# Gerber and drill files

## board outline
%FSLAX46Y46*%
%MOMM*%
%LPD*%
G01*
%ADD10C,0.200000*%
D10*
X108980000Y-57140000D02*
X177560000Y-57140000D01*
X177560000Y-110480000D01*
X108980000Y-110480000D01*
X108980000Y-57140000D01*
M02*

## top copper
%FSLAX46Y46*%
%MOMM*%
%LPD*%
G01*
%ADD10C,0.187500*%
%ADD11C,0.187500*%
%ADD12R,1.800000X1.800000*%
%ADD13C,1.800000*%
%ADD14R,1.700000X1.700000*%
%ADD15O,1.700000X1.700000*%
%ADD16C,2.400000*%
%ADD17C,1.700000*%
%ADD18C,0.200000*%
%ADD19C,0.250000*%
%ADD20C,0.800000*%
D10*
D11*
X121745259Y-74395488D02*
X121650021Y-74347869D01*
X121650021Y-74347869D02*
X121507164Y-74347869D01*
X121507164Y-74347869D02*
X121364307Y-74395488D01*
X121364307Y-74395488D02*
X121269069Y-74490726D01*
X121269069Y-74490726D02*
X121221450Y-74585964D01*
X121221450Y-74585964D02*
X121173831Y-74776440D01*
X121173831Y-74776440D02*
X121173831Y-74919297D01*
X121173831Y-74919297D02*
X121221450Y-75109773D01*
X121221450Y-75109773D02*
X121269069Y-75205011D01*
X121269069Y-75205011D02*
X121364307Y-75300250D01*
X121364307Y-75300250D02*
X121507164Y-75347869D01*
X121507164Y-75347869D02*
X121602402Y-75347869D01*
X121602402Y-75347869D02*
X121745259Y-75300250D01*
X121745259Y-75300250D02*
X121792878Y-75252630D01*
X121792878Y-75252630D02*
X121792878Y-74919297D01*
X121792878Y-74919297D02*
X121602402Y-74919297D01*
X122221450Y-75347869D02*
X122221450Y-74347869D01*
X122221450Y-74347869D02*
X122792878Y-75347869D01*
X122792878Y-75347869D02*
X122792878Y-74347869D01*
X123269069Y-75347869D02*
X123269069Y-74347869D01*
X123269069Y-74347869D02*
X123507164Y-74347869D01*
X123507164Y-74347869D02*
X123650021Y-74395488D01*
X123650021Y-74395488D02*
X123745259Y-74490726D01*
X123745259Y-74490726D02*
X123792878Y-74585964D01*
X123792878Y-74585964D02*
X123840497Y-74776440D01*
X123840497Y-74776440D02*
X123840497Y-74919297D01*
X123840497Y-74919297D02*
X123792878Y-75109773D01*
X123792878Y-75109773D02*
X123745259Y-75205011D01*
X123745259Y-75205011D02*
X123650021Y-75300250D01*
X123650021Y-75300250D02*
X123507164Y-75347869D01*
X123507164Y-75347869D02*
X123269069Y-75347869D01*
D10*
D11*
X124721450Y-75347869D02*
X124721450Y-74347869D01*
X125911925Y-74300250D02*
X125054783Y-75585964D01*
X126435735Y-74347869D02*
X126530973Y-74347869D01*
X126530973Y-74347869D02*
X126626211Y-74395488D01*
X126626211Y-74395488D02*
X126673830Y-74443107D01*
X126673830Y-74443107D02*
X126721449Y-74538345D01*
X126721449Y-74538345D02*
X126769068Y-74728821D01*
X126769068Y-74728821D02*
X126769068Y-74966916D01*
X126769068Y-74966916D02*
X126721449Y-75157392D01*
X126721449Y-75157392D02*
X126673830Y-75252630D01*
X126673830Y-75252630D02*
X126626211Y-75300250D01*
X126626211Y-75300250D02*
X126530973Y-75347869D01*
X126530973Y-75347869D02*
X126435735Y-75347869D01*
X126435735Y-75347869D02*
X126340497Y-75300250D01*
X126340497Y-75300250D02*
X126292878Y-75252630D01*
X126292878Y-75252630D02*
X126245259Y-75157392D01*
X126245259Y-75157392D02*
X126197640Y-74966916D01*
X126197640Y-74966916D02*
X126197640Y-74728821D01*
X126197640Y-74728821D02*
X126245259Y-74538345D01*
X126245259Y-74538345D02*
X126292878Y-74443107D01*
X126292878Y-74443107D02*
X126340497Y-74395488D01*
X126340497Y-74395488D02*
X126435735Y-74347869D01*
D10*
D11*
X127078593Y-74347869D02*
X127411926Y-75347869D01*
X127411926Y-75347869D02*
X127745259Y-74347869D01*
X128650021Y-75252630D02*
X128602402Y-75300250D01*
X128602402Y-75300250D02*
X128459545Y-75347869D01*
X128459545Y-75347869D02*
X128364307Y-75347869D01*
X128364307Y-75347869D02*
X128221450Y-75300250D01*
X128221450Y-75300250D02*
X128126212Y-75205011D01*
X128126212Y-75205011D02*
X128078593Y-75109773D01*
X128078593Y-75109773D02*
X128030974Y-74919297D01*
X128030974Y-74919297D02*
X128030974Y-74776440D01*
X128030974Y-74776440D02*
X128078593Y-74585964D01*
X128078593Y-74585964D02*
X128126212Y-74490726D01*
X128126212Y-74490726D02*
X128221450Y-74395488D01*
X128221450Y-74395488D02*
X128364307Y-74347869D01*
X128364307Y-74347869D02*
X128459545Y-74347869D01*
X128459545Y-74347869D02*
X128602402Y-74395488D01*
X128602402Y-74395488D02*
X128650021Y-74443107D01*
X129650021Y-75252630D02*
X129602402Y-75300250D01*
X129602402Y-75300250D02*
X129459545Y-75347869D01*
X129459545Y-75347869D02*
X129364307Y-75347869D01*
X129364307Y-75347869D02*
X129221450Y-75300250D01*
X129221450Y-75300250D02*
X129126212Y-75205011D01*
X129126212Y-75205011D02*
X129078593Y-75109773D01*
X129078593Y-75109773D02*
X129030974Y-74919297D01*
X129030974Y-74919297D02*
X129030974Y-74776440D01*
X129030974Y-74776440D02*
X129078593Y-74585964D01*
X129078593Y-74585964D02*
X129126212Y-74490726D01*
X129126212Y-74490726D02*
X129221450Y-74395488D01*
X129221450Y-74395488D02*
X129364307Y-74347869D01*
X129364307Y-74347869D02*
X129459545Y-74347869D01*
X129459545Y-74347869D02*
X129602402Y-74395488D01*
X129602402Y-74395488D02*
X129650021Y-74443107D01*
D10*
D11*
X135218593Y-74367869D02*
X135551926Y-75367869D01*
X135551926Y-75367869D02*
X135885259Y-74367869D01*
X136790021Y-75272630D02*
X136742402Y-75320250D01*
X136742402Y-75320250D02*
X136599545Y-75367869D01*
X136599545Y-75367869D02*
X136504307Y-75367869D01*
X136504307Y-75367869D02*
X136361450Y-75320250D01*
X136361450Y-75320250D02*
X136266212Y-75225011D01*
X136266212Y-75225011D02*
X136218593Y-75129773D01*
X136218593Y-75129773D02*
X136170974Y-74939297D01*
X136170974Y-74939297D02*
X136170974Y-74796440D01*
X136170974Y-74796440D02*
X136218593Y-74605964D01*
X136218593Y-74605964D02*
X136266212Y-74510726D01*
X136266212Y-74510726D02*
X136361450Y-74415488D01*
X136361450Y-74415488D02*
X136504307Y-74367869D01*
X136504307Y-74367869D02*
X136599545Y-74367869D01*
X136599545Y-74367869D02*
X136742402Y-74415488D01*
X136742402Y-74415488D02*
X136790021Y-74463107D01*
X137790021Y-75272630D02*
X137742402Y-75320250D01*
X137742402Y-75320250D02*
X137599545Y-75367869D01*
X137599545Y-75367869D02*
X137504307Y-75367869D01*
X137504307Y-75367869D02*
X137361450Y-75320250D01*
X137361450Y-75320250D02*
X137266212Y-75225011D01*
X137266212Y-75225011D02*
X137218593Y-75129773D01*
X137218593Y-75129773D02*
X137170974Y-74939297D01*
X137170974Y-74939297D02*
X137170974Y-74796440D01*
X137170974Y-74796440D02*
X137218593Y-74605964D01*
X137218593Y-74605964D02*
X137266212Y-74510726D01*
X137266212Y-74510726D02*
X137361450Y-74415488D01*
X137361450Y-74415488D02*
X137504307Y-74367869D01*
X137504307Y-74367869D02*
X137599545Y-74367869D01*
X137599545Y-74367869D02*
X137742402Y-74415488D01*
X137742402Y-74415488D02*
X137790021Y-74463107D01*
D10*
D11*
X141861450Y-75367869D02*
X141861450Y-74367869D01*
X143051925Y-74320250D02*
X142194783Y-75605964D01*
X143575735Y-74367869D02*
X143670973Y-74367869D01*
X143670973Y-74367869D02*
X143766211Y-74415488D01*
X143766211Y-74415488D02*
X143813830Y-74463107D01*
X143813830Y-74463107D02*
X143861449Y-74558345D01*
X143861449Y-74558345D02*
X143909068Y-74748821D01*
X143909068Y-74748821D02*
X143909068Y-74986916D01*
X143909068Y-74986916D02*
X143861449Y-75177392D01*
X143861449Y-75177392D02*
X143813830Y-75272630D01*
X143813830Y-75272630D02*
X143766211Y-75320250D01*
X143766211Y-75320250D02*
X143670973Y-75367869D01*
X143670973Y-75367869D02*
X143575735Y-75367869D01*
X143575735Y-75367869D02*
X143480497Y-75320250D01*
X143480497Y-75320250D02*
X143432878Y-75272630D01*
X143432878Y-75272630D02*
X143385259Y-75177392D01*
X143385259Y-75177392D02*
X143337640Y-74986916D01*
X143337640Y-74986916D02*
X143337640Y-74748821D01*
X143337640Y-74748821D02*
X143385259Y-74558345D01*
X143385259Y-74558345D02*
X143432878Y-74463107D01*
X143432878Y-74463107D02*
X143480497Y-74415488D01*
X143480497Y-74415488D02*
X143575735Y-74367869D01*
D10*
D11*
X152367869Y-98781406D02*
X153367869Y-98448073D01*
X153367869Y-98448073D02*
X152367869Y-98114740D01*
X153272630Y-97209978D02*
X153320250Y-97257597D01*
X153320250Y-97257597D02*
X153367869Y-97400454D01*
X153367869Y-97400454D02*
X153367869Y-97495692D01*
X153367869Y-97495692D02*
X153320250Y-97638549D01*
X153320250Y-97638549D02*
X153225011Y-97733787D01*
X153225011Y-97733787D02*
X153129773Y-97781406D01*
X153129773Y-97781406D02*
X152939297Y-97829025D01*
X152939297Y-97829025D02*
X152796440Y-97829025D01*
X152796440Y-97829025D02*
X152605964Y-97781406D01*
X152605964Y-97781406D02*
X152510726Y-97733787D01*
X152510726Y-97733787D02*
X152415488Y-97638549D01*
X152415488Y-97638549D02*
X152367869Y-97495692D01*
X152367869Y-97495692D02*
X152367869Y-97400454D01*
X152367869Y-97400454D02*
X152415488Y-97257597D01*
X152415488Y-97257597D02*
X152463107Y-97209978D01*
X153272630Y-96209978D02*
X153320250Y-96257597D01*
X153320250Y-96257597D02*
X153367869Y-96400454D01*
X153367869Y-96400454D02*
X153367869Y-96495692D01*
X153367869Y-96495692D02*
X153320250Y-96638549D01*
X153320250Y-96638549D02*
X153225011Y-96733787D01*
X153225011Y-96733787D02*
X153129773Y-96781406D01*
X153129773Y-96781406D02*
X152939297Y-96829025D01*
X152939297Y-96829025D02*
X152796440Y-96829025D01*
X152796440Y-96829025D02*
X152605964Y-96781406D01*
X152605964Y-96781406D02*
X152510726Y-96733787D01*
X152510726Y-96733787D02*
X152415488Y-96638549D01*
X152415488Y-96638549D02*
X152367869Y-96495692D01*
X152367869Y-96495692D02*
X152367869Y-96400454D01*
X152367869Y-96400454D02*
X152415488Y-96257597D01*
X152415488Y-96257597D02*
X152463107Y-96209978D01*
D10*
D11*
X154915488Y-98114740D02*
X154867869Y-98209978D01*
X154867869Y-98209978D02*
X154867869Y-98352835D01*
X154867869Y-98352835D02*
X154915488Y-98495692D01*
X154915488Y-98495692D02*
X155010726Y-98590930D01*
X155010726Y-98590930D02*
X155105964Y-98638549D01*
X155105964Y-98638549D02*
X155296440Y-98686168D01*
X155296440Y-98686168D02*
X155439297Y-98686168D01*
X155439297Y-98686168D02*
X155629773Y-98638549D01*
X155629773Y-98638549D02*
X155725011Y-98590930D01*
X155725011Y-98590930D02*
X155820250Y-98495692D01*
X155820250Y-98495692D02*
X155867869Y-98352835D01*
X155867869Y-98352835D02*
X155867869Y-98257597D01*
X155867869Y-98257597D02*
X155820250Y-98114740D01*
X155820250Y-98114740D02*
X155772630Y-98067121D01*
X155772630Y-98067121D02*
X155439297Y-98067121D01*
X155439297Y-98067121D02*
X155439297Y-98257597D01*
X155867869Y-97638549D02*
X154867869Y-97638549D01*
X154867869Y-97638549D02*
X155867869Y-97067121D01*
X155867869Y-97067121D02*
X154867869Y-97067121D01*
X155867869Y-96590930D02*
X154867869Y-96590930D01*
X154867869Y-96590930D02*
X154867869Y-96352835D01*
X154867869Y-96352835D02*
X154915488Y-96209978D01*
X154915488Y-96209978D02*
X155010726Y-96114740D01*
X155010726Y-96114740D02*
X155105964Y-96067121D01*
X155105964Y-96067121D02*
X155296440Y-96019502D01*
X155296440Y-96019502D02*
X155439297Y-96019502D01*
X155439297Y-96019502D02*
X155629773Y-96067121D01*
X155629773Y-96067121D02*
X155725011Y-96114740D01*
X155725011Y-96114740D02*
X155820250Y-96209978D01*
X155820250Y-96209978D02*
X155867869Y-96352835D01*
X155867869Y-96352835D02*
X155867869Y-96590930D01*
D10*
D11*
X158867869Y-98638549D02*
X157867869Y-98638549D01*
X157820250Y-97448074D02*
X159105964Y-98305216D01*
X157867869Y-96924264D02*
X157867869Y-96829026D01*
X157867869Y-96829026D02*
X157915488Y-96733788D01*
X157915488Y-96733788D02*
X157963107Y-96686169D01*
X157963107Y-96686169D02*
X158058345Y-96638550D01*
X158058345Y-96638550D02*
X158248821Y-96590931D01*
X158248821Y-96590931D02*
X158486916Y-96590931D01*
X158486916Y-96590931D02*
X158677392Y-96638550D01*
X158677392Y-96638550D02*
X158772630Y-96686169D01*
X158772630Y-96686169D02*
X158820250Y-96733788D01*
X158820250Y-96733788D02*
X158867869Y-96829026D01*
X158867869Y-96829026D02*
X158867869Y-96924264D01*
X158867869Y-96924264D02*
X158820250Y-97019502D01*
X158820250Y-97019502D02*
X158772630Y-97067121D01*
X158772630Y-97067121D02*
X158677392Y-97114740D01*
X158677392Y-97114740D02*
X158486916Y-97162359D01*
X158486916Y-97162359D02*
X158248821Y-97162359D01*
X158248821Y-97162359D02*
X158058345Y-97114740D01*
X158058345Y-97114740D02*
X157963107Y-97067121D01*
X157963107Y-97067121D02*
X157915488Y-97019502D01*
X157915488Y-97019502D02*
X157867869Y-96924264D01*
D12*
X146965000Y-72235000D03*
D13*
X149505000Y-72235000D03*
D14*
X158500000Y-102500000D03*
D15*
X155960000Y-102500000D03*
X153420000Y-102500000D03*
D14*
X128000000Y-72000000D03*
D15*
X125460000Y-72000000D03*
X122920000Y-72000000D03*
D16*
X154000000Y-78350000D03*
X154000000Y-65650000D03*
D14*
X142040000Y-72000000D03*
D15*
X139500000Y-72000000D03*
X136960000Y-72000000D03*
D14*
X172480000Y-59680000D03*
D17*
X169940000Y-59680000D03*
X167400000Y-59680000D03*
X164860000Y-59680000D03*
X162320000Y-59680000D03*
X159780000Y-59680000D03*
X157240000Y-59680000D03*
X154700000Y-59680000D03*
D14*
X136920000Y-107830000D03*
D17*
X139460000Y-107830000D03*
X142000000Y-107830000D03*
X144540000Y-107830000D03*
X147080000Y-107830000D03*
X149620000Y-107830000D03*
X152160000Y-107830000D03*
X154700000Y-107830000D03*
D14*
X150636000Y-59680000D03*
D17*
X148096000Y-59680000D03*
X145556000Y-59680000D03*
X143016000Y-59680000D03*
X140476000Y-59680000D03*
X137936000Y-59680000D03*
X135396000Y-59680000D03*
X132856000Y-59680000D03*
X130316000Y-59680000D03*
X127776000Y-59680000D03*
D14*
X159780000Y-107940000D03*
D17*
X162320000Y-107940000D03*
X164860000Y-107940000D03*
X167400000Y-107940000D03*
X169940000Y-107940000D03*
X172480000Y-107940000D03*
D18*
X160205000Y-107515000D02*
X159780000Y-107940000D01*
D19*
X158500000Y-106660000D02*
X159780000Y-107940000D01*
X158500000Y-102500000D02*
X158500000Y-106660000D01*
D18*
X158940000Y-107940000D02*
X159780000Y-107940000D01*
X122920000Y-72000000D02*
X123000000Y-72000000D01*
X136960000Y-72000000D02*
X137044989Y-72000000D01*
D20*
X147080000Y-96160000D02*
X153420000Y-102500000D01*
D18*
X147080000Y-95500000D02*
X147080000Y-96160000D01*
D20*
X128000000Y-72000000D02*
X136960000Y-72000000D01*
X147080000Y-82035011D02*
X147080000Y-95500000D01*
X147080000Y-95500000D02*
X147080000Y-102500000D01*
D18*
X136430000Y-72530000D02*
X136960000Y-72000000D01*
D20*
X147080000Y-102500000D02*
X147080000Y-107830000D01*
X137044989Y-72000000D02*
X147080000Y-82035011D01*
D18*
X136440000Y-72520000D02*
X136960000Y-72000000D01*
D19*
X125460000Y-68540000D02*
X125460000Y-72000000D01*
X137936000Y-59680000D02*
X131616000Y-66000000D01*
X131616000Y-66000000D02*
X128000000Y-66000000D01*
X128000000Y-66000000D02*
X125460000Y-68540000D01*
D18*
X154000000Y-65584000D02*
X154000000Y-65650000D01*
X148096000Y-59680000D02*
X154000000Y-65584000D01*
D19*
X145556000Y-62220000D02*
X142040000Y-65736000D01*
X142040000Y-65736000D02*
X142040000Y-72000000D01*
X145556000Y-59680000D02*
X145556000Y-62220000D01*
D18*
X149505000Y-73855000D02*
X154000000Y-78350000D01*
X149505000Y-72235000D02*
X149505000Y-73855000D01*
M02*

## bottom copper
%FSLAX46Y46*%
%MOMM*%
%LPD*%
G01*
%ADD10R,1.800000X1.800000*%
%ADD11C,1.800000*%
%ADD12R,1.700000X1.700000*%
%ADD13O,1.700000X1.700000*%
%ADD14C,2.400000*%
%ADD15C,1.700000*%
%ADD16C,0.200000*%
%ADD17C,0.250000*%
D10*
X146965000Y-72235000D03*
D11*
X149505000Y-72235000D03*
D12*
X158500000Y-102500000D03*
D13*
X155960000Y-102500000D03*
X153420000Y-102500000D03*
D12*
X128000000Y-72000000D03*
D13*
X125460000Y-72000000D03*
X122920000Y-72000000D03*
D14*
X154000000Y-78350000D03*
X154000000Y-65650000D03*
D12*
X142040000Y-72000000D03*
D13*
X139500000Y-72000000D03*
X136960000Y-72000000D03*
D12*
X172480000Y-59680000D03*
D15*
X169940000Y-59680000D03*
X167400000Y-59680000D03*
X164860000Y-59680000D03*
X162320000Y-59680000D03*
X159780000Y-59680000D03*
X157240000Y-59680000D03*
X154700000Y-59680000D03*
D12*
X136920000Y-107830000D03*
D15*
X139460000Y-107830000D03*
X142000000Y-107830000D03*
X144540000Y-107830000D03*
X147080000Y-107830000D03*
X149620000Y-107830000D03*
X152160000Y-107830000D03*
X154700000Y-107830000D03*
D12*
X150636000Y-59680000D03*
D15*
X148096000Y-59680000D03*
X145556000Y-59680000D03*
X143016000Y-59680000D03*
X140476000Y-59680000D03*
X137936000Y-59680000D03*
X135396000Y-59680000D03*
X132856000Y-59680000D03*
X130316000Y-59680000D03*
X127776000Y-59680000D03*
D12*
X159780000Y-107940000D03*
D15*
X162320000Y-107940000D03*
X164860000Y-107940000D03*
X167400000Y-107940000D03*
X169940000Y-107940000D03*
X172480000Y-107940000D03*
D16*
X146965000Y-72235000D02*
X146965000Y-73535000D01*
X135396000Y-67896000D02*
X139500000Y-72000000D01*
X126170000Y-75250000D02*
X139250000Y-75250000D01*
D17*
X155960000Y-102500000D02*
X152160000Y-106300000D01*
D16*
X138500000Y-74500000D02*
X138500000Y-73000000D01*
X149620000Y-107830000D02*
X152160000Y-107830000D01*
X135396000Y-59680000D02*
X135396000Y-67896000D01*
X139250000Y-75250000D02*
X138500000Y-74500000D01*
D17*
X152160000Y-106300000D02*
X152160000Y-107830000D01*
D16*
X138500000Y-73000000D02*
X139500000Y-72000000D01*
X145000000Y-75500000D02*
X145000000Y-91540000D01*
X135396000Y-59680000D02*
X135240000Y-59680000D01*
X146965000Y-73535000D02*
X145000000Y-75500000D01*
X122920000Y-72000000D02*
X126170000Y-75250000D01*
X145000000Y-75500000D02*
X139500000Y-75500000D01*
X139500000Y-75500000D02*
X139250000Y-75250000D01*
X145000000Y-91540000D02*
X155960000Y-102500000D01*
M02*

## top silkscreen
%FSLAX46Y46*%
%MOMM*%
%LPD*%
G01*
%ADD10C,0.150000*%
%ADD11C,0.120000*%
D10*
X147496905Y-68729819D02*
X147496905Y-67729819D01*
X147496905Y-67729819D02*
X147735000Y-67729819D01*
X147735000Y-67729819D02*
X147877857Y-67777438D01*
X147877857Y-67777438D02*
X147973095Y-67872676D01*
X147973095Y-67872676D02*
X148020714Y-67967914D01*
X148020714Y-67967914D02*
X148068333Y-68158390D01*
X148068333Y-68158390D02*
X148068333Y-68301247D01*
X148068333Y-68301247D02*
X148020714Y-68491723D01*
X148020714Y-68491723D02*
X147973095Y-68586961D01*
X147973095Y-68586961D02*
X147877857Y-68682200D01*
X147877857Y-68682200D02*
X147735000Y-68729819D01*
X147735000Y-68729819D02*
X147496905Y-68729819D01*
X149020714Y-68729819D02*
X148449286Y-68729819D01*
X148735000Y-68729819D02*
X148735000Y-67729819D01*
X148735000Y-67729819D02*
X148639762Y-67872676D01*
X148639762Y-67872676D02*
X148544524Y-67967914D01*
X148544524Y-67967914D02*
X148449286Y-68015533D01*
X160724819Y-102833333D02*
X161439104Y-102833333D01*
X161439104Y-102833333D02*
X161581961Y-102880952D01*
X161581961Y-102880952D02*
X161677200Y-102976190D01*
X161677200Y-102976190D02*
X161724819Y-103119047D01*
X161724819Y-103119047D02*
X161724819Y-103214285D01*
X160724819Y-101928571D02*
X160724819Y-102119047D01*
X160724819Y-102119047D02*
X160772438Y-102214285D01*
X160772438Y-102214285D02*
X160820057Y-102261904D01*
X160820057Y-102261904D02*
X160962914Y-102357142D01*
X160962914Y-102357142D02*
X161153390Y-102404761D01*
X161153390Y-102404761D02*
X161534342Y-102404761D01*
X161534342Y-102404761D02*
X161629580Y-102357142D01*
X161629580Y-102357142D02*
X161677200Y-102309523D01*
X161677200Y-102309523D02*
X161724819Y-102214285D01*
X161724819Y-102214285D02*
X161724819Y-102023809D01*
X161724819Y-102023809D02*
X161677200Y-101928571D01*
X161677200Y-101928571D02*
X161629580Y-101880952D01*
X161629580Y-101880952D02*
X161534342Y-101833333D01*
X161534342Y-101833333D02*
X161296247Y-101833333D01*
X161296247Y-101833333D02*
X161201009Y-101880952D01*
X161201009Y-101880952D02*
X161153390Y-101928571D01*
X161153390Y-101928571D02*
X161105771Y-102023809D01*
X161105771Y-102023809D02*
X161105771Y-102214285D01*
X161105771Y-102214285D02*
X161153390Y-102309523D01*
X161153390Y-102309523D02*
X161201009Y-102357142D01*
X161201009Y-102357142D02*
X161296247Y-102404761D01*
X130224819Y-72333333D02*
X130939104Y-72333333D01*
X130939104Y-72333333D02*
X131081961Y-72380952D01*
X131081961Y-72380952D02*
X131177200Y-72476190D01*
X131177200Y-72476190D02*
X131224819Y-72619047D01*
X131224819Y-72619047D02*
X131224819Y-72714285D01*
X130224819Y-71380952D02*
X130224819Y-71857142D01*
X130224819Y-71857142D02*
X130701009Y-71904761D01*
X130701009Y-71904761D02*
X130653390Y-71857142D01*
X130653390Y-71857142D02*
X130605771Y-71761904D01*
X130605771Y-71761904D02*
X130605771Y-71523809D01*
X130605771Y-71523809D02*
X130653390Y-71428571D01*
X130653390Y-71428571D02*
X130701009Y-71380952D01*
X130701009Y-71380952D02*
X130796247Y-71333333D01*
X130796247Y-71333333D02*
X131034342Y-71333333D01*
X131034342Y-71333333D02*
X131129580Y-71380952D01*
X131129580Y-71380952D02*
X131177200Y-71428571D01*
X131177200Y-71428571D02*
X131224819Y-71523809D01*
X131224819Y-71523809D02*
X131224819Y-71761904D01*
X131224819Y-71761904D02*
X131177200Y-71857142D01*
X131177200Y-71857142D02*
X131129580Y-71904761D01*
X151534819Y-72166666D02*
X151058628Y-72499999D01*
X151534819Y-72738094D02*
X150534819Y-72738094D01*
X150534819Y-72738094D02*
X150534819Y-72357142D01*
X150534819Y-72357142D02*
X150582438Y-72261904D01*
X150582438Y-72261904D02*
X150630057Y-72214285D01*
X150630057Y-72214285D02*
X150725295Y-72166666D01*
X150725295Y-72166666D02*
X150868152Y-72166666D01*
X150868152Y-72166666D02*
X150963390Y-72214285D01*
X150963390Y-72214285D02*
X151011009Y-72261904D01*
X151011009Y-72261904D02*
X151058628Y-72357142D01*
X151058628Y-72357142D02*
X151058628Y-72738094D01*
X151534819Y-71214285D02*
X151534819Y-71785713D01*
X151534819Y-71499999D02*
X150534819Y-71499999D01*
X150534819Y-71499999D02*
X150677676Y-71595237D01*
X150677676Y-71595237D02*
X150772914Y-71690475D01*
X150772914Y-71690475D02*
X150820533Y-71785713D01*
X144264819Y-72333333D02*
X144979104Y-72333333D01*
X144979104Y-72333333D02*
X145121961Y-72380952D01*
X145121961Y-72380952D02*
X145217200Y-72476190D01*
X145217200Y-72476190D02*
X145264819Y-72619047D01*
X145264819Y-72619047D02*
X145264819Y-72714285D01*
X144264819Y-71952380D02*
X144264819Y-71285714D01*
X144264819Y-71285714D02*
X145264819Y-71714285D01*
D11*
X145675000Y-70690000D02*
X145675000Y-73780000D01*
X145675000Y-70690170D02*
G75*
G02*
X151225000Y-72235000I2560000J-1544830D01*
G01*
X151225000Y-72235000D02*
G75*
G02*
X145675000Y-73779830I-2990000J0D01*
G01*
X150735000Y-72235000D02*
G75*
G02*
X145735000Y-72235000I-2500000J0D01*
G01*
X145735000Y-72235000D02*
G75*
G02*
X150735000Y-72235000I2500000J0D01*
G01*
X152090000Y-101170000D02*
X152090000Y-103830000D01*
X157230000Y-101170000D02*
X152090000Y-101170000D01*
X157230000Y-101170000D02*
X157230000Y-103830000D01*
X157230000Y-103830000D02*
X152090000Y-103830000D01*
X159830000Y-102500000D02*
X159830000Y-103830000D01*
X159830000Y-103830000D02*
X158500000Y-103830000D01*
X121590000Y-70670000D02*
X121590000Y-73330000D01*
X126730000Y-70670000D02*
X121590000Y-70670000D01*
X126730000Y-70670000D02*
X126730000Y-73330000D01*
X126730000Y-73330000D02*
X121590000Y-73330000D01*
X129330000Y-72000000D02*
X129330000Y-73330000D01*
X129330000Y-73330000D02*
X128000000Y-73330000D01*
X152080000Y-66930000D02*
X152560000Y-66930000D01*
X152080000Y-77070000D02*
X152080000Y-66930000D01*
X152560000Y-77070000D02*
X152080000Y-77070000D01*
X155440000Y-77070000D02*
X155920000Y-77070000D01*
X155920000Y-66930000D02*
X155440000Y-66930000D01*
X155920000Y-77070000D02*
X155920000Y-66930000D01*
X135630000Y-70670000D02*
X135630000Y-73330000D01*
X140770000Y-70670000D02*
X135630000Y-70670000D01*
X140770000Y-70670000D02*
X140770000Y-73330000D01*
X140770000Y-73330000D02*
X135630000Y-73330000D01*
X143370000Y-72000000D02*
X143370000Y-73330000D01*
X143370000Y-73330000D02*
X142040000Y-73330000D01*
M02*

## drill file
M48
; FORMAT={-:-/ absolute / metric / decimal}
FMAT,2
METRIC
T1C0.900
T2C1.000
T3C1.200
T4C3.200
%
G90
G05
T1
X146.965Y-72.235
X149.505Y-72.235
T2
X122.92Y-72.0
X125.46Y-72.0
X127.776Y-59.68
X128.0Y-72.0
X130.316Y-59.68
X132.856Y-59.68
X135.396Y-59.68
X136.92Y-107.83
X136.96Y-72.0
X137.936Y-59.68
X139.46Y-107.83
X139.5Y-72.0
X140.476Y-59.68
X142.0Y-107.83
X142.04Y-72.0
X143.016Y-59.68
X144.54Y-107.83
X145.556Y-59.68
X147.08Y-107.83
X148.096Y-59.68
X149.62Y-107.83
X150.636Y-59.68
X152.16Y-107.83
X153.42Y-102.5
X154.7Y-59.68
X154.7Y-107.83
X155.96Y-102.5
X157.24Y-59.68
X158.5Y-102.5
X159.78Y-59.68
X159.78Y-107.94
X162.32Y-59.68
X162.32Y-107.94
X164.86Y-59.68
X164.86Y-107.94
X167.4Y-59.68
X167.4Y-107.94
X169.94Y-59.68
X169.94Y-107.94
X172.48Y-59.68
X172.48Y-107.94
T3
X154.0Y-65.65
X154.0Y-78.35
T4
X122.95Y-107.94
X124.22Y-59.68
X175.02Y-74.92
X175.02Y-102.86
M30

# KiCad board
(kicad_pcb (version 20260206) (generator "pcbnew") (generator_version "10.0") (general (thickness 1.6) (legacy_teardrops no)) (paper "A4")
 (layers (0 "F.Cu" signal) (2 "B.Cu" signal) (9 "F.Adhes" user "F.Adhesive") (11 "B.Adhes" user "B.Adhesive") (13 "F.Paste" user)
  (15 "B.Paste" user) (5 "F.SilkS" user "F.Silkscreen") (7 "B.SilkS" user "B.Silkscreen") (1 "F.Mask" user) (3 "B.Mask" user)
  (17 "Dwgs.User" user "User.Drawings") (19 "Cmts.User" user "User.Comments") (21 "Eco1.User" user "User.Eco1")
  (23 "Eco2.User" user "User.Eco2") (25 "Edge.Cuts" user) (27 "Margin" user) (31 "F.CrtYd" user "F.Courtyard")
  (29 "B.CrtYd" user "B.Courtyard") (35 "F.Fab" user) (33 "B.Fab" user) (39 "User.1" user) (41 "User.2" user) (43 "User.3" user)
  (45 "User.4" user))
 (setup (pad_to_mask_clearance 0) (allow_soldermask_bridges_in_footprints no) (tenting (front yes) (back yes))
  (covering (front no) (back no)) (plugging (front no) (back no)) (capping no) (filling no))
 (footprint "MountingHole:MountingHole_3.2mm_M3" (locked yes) (layer "F.Cu") (at 175.01997 102.860094)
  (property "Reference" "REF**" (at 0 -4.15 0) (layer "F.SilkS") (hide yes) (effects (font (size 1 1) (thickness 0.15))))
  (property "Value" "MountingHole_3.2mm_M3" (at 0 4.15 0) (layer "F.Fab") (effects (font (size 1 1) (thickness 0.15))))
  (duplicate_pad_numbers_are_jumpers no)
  (pad "" np_thru_hole circle (at 0 0) (size 3.2 3.2) (drill 3.2) (layers "*.Cu" "*.Mask")))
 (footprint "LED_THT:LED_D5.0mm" (layer "F.Cu") (at 146.965 72.235)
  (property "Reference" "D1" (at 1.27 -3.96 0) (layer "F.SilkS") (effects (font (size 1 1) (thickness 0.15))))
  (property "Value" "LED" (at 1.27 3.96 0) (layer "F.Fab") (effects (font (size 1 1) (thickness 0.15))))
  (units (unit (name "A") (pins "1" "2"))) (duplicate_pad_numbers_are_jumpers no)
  (fp_line (start -1.29 -1.545) (end -1.29 1.545) (stroke (width 0.12) (type solid)) (layer "F.SilkS"))
  (fp_arc (start -1.29 -1.54483) (mid 2.071779 -2.880495) (end 4.26 0) (stroke (width 0.12) (type solid)) (layer "F.SilkS"))
  (fp_arc (start 4.26 0) (mid 2.071779 2.880495) (end -1.29 1.54483) (stroke (width 0.12) (type solid)) (layer "F.SilkS"))
  (fp_circle (center 1.27 0) (end 3.77 0) (stroke (width 0.12) (type solid)) (fill no) (layer "F.SilkS"))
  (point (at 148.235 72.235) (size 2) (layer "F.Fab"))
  (pad "1" thru_hole rect (at 0 0) (size 1.8 1.8) (drill 0.9) (layers "*.Cu" "*.Mask") (remove_unused_layers no) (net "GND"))
  (pad "2" thru_hole circle (at 2.54 0) (size 1.8 1.8) (drill 0.9) (layers "*.Cu" "*.Mask") (remove_unused_layers no) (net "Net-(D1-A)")))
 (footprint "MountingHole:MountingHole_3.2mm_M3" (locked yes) (layer "F.Cu") (at 122.94997 107.940094)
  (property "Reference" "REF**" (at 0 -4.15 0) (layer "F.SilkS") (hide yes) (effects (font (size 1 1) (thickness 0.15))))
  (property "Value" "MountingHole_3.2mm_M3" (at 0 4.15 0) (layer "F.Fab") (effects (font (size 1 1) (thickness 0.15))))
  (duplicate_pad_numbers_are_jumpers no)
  (pad "" np_thru_hole circle (at 0 0) (size 3.2 3.2) (drill 3.2) (layers "*.Cu" "*.Mask")))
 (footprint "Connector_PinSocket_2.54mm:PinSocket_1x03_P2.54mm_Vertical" (layer "F.Cu") (at 158.5 102.5 -90)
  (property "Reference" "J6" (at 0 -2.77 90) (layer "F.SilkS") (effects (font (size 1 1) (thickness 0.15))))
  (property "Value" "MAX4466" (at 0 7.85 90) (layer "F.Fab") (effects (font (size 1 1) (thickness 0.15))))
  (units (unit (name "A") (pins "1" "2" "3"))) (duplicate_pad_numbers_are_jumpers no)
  (fp_line (start -1.33 6.41) (end 1.33 6.41) (stroke (width 0.12) (type solid)) (layer "F.SilkS"))
  (fp_line (start -1.33 1.27) (end -1.33 6.41) (stroke (width 0.12) (type solid)) (layer "F.SilkS"))
  (fp_line (start -1.33 1.27) (end 1.33 1.27) (stroke (width 0.12) (type solid)) (layer "F.SilkS"))
  (fp_line (start 1.33 1.27) (end 1.33 6.41) (stroke (width 0.12) (type solid)) (layer "F.SilkS"))
  (fp_line (start 0 -1.33) (end 1.33 -1.33) (stroke (width 0.12) (type solid)) (layer "F.SilkS"))
  (fp_line (start 1.33 -1.33) (end 1.33 0) (stroke (width 0.12) (type solid)) (layer "F.SilkS"))
  (pad "1" thru_hole rect (at 0 0 270) (size 1.7 1.7) (drill 1) (layers "*.Cu" "*.Mask") (remove_unused_layers no) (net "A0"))
  (pad "2" thru_hole oval (at 0 2.54 270) (size 1.7 1.7) (drill 1) (layers "*.Cu" "*.Mask") (remove_unused_layers no) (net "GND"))
  (pad "3" thru_hole oval (at 0 5.08 270) (size 1.7 1.7) (drill 1) (layers "*.Cu" "*.Mask") (remove_unused_layers no) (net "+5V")))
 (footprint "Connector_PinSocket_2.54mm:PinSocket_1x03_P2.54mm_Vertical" (layer "F.Cu") (at 128 72 -90)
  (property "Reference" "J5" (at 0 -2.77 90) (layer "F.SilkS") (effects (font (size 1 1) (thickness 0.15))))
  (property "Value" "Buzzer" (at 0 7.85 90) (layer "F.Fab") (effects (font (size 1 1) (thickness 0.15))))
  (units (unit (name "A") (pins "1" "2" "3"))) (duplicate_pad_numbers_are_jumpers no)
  (fp_line (start -1.33 6.41) (end 1.33 6.41) (stroke (width 0.12) (type solid)) (layer "F.SilkS"))
  (fp_line (start -1.33 1.27) (end -1.33 6.41) (stroke (width 0.12) (type solid)) (layer "F.SilkS"))
  (fp_line (start -1.33 1.27) (end 1.33 1.27) (stroke (width 0.12) (type solid)) (layer "F.SilkS"))
  (fp_line (start 1.33 1.27) (end 1.33 6.41) (stroke (width 0.12) (type solid)) (layer "F.SilkS"))
  (fp_line (start 0 -1.33) (end 1.33 -1.33) (stroke (width 0.12) (type solid)) (layer "F.SilkS"))
  (fp_line (start 1.33 -1.33) (end 1.33 0) (stroke (width 0.12) (type solid)) (layer "F.SilkS"))
  (pad "1" thru_hole rect (at 0 0 270) (size 1.7 1.7) (drill 1) (layers "*.Cu" "*.Mask") (remove_unused_layers no) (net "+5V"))
  (pad "2" thru_hole oval (at 0 2.54 270) (size 1.7 1.7) (drill 1) (layers "*.Cu" "*.Mask") (remove_unused_layers no) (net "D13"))
  (pad "3" thru_hole oval (at 0 5.08 270) (size 1.7 1.7) (drill 1) (layers "*.Cu" "*.Mask") (remove_unused_layers no) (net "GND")))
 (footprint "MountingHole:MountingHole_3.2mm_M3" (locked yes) (layer "F.Cu") (at 124.21997 59.680094)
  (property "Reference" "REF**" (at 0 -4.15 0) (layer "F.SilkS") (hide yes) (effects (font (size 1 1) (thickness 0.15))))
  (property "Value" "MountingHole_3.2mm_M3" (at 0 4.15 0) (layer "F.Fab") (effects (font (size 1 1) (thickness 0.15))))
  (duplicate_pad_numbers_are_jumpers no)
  (pad "" np_thru_hole circle (at 0 0) (size 3.2 3.2) (drill 3.2) (layers "*.Cu" "*.Mask")))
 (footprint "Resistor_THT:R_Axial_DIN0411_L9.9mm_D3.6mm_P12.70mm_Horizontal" (layer "F.Cu") (at 154 78.35 90)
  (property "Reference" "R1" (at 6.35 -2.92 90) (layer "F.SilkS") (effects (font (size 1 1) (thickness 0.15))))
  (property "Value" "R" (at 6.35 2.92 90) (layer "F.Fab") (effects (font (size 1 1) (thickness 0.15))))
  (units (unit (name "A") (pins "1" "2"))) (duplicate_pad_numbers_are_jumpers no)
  (fp_line (start 11.42 -1.92) (end 11.42 -1.44) (stroke (width 0.12) (type solid)) (layer "F.SilkS"))
  (fp_line (start 1.28 -1.92) (end 11.42 -1.92) (stroke (width 0.12) (type solid)) (layer "F.SilkS"))
  (fp_line (start 1.28 -1.44) (end 1.28 -1.92) (stroke (width 0.12) (type solid)) (layer "F.SilkS"))
  (fp_line (start 1.28 1.44) (end 1.28 1.92) (stroke (width 0.12) (type solid)) (layer "F.SilkS"))
  (fp_line (start 11.42 1.92) (end 11.42 1.44) (stroke (width 0.12) (type solid)) (layer "F.SilkS"))
  (fp_line (start 1.28 1.92) (end 11.42 1.92) (stroke (width 0.12) (type solid)) (layer "F.SilkS"))
  (pad "1" thru_hole circle (at 0 0 90) (size 2.4 2.4) (drill 1.2) (layers "*.Cu" "*.Mask") (remove_unused_layers no) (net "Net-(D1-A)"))
  (pad "2" thru_hole circle (at 12.7 0 90) (size 2.4 2.4) (drill 1.2) (layers "*.Cu" "*.Mask") (remove_unused_layers no) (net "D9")))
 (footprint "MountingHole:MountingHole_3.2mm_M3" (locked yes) (layer "F.Cu") (at 175.01997 74.920094)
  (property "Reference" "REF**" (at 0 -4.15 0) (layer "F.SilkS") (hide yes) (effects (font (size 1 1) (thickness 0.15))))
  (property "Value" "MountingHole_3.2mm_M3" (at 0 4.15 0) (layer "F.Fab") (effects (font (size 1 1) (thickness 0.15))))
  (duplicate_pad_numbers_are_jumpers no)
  (pad "" np_thru_hole circle (at 0 0) (size 3.2 3.2) (drill 3.2) (layers "*.Cu" "*.Mask")))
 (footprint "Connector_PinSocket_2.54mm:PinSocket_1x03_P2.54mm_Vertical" (layer "F.Cu") (at 142.04 72 -90)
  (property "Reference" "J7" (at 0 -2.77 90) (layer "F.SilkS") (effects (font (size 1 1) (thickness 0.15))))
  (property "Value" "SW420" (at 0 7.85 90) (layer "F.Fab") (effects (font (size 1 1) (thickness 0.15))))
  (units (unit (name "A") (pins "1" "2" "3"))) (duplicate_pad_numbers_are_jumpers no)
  (fp_line (start -1.33 6.41) (end 1.33 6.41) (stroke (width 0.12) (type solid)) (layer "F.SilkS"))
  (fp_line (start -1.33 1.27) (end -1.33 6.41) (stroke (width 0.12) (type solid)) (layer "F.SilkS"))
  (fp_line (start -1.33 1.27) (end 1.33 1.27) (stroke (width 0.12) (type solid)) (layer "F.SilkS"))
  (fp_line (start 1.33 1.27) (end 1.33 6.41) (stroke (width 0.12) (type solid)) (layer "F.SilkS"))
  (fp_line (start 0 -1.33) (end 1.33 -1.33) (stroke (width 0.12) (type solid)) (layer "F.SilkS"))
  (fp_line (start 1.33 -1.33) (end 1.33 0) (stroke (width 0.12) (type solid)) (layer "F.SilkS"))
  (pad "1" thru_hole rect (at 0 0 270) (size 1.7 1.7) (drill 1) (layers "*.Cu" "*.Mask") (remove_unused_layers no) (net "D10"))
  (pad "2" thru_hole oval (at 0 2.54 270) (size 1.7 1.7) (drill 1) (layers "*.Cu" "*.Mask") (remove_unused_layers no) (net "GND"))
  (pad "3" thru_hole oval (at 0 5.08 270) (size 1.7 1.7) (drill 1) (layers "*.Cu" "*.Mask") (remove_unused_layers no) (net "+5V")))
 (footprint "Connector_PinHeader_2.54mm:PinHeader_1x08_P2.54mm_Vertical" (layer "B.Cu") (at 172.48 59.68 90)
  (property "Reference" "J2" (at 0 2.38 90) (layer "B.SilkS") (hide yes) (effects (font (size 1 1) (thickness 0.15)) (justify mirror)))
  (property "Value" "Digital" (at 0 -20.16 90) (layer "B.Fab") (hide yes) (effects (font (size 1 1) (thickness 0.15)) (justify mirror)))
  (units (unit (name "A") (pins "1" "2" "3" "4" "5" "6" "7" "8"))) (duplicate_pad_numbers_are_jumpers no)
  (pad "1" thru_hole rect (at 0 0 90) (size 1.7 1.7) (drill 1) (layers "*.Cu" "*.Mask") (remove_unused_layers no) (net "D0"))
  (pad "2" thru_hole circle (at 0 -2.54 90) (size 1.7 1.7) (drill 1) (layers "*.Cu" "*.Mask") (remove_unused_layers no) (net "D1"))
  (pad "3" thru_hole circle (at 0 -5.08 90) (size 1.7 1.7) (drill 1) (layers "*.Cu" "*.Mask") (remove_unused_layers no) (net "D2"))
  (pad "4" thru_hole circle (at 0 -7.62 90) (size 1.7 1.7) (drill 1) (layers "*.Cu" "*.Mask") (remove_unused_layers no) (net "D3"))
  (pad "5" thru_hole circle (at 0 -10.16 90) (size 1.7 1.7) (drill 1) (layers "*.Cu" "*.Mask") (remove_unused_layers no) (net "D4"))
  (pad "6" thru_hole circle (at 0 -12.7 90) (size 1.7 1.7) (drill 1) (layers "*.Cu" "*.Mask") (remove_unused_layers no) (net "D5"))
  (pad "7" thru_hole circle (at 0 -15.24 90) (size 1.7 1.7) (drill 1) (layers "*.Cu" "*.Mask") (remove_unused_layers no) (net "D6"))
  (pad "8" thru_hole circle (at 0 -17.78 90) (size 1.7 1.7) (drill 1) (layers "*.Cu" "*.Mask") (remove_unused_layers no) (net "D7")))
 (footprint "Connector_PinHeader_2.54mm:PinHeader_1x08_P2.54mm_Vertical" (layer "B.Cu") (at 136.92 107.83 -90)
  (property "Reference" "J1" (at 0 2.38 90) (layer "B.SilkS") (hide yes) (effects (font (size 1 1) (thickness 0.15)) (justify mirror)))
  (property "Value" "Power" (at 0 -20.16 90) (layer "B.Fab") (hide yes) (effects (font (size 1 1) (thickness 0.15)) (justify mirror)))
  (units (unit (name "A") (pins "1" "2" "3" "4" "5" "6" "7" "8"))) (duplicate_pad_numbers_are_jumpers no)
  (pad "1" thru_hole rect (at 0 0 270) (size 1.7 1.7) (drill 1) (layers "*.Cu" "*.Mask") (remove_unused_layers no)
   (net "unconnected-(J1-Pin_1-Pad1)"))
  (pad "2" thru_hole circle (at 0 -2.54 270) (size 1.7 1.7) (drill 1) (layers "*.Cu" "*.Mask") (remove_unused_layers no) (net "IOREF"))
  (pad "3" thru_hole circle (at 0 -5.08 270) (size 1.7 1.7) (drill 1) (layers "*.Cu" "*.Mask") (remove_unused_layers no) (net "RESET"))
  (pad "4" thru_hole circle (at 0 -7.62 270) (size 1.7 1.7) (drill 1) (layers "*.Cu" "*.Mask") (remove_unused_layers no) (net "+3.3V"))
  (pad "5" thru_hole circle (at 0 -10.16 270) (size 1.7 1.7) (drill 1) (layers "*.Cu" "*.Mask") (remove_unused_layers no) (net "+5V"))
  (pad "6" thru_hole circle (at 0 -12.7 270) (size 1.7 1.7) (drill 1) (layers "*.Cu" "*.Mask") (remove_unused_layers no) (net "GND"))
  (pad "7" thru_hole circle (at 0 -15.24 270) (size 1.7 1.7) (drill 1) (layers "*.Cu" "*.Mask") (remove_unused_layers no) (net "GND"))
  (pad "8" thru_hole circle (at 0 -17.78 270) (size 1.7 1.7) (drill 1) (layers "*.Cu" "*.Mask") (remove_unused_layers no) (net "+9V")))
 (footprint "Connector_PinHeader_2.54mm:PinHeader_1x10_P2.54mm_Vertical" (layer "B.Cu") (at 150.636 59.68 90)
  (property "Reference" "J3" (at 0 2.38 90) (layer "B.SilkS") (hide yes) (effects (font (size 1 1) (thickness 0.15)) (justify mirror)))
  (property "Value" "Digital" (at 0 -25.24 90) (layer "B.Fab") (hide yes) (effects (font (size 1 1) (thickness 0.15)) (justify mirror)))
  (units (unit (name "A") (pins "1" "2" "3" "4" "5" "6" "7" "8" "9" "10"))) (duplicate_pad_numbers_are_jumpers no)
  (pad "1" thru_hole rect (at 0 0 90) (size 1.7 1.7) (drill 1) (layers "*.Cu" "*.Mask") (remove_unused_layers no) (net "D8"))
  (pad "2" thru_hole circle (at 0 -2.54 90) (size 1.7 1.7) (drill 1) (layers "*.Cu" "*.Mask") (remove_unused_layers no) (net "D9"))
  (pad "3" thru_hole circle (at 0 -5.08 90) (size 1.7 1.7) (drill 1) (layers "*.Cu" "*.Mask") (remove_unused_layers no) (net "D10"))
  (pad "4" thru_hole circle (at 0 -7.62 90) (size 1.7 1.7) (drill 1) (layers "*.Cu" "*.Mask") (remove_unused_layers no) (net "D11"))
  (pad "5" thru_hole circle (at 0 -10.16 90) (size 1.7 1.7) (drill 1) (layers "*.Cu" "*.Mask") (remove_unused_layers no) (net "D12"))
  (pad "6" thru_hole circle (at 0 -12.7 90) (size 1.7 1.7) (drill 1) (layers "*.Cu" "*.Mask") (remove_unused_layers no) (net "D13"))
  (pad "7" thru_hole circle (at 0 -15.24 90) (size 1.7 1.7) (drill 1) (layers "*.Cu" "*.Mask") (remove_unused_layers no) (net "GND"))
  (pad "8" thru_hole circle (at 0 -17.78 90) (size 1.7 1.7) (drill 1) (layers "*.Cu" "*.Mask") (remove_unused_layers no)
   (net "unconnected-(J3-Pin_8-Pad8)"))
  (pad "9" thru_hole circle (at 0 -20.32 90) (size 1.7 1.7) (drill 1) (layers "*.Cu" "*.Mask") (remove_unused_layers no)
   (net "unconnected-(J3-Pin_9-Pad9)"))
  (pad "10" thru_hole circle (at 0 -22.86 90) (size 1.7 1.7) (drill 1) (layers "*.Cu" "*.Mask") (remove_unused_layers no)
   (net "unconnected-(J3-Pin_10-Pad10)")))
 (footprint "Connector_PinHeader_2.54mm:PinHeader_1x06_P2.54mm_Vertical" (layer "B.Cu") (at 159.78 107.94 -90)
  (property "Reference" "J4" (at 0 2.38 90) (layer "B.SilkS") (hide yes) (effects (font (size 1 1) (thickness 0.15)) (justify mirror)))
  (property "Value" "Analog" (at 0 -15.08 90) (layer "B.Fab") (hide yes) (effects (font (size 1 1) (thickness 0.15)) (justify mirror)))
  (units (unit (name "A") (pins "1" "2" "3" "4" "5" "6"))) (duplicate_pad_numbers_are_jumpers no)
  (pad "1" thru_hole rect (at 0 0 270) (size 1.7 1.7) (drill 1) (layers "*.Cu" "*.Mask") (remove_unused_layers no) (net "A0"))
  (pad "2" thru_hole circle (at 0 -2.54 270) (size 1.7 1.7) (drill 1) (layers "*.Cu" "*.Mask") (remove_unused_layers no) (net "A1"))
  (pad "3" thru_hole circle (at 0 -5.08 270) (size 1.7 1.7) (drill 1) (layers "*.Cu" "*.Mask") (remove_unused_layers no) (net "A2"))
  (pad "4" thru_hole circle (at 0 -7.62 270) (size 1.7 1.7) (drill 1) (layers "*.Cu" "*.Mask") (remove_unused_layers no) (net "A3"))
  (pad "5" thru_hole circle (at 0 -10.16 270) (size 1.7 1.7) (drill 1) (layers "*.Cu" "*.Mask") (remove_unused_layers no) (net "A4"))
  (pad "6" thru_hole circle (at 0 -12.7 270) (size 1.7 1.7) (drill 1) (layers "*.Cu" "*.Mask") (remove_unused_layers no) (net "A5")))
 (gr_rect (start 108.98 57.14) (end 177.56 110.48) (stroke (width 0.2) (type solid)) (fill no) (layer "Edge.Cuts"))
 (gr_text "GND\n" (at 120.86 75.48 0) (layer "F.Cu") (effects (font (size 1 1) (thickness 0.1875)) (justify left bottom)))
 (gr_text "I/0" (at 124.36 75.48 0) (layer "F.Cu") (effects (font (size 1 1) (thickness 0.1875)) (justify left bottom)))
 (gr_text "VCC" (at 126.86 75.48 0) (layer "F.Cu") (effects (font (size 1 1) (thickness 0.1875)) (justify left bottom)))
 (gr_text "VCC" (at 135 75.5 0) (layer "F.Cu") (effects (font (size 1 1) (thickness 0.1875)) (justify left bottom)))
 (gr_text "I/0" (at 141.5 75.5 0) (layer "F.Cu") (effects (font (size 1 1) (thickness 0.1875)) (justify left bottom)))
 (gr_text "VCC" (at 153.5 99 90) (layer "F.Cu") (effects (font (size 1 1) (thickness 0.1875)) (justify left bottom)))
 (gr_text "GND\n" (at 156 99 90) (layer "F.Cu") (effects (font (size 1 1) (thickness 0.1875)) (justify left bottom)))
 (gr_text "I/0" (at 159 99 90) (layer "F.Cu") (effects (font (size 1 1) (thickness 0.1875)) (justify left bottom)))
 (segment (start 160.205 107.515) (end 159.78 107.94) (width 0.2) (layer "F.Cu") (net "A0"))
 (segment (start 158.5 106.66) (end 159.78 107.94) (width 0.25) (layer "F.Cu") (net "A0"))
 (segment (start 158.5 102.5) (end 158.5 106.66) (width 0.25) (layer "F.Cu") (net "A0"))
 (segment (start 158.94 107.94) (end 159.78 107.94) (width 0.2) (layer "F.Cu") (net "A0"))
 (segment (start 122.92 72) (end 123 72) (width 0.2) (layer "F.Cu") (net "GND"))
 (segment (start 146.965 72.235) (end 146.965 73.535) (width 0.2) (layer "B.Cu") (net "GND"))
 (segment (start 135.396 67.896) (end 139.5 72) (width 0.2) (layer "B.Cu") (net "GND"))
 (segment (start 126.17 75.25) (end 139.25 75.25) (width 0.2) (layer "B.Cu") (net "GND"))
 (segment (start 155.96 102.5) (end 152.16 106.3) (width 0.25) (layer "B.Cu") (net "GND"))
 (segment (start 138.5 74.5) (end 138.5 73) (width 0.2) (layer "B.Cu") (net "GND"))
 (segment (start 149.62 107.83) (end 152.16 107.83) (width 0.2) (layer "B.Cu") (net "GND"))
 (segment (start 135.396 59.68) (end 135.396 67.896) (width 0.2) (layer "B.Cu") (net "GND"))
 (segment (start 139.25 75.25) (end 138.5 74.5) (width 0.2) (layer "B.Cu") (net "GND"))
 (segment (start 152.16 106.3) (end 152.16 107.83) (width 0.25) (layer "B.Cu") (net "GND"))
 (segment (start 138.5 73) (end 139.5 72) (width 0.2) (layer "B.Cu") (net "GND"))
 (segment (start 145 75.5) (end 145 91.54) (width 0.2) (layer "B.Cu") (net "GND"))
 (segment (start 135.396 59.68) (end 135.24 59.68) (width 0.2) (layer "B.Cu") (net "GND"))
 (segment (start 146.965 73.535) (end 145 75.5) (width 0.2) (layer "B.Cu") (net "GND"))
 (segment (start 122.92 72) (end 126.17 75.25) (width 0.2) (layer "B.Cu") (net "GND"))
 (segment (start 145 75.5) (end 139.5 75.5) (width 0.2) (layer "B.Cu") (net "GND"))
 (segment (start 139.5 75.5) (end 139.25 75.25) (width 0.2) (layer "B.Cu") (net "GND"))
 (segment (start 145 91.54) (end 155.96 102.5) (width 0.2) (layer "B.Cu") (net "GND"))
 (segment (start 136.96 72) (end 137.044989 72) (width 0.2) (layer "F.Cu") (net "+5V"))
 (segment (start 147.08 96.16) (end 153.42 102.5) (width 0.8) (layer "F.Cu") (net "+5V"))
 (segment (start 147.08 95.5) (end 147.08 96.16) (width 0.2) (layer "F.Cu") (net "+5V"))
 (segment (start 128 72) (end 136.96 72) (width 0.8) (layer "F.Cu") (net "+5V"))
 (segment (start 147.08 82.035011) (end 147.08 95.5) (width 0.8) (layer "F.Cu") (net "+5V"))
 (segment (start 147.08 95.5) (end 147.08 102.5) (width 0.8) (layer "F.Cu") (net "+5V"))
 (segment (start 136.43 72.53) (end 136.96 72) (width 0.2) (layer "F.Cu") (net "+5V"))
 (segment (start 147.08 102.5) (end 147.08 107.83) (width 0.8) (layer "F.Cu") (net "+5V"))
 (segment (start 137.044989 72) (end 147.08 82.035011) (width 0.8) (layer "F.Cu") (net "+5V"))
 (segment (start 136.44 72.52) (end 136.96 72) (width 0.2) (layer "F.Cu") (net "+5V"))
 (segment (start 125.46 68.54) (end 125.46 72) (width 0.25) (layer "F.Cu") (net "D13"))
 (segment (start 137.936 59.68) (end 131.616 66) (width 0.25) (layer "F.Cu") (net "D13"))
 (segment (start 131.616 66) (end 128 66) (width 0.25) (layer "F.Cu") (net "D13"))
 (segment (start 128 66) (end 125.46 68.54) (width 0.25) (layer "F.Cu") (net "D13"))
 (segment (start 154 65.584) (end 154 65.65) (width 0.2) (layer "F.Cu") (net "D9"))
 (segment (start 148.096 59.68) (end 154 65.584) (width 0.2) (layer "F.Cu") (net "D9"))
 (segment (start 145.556 62.22) (end 142.04 65.736) (width 0.25) (layer "F.Cu") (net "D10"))
 (segment (start 142.04 65.736) (end 142.04 72) (width 0.25) (layer "F.Cu") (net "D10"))
 (segment (start 145.556 59.68) (end 145.556 62.22) (width 0.25) (layer "F.Cu") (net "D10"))
 (segment (start 149.505 73.855) (end 154 78.35) (width 0.2) (layer "F.Cu") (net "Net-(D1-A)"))
 (segment (start 149.505 72.235) (end 149.505 73.855) (width 0.2) (layer "F.Cu") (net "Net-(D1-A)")))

